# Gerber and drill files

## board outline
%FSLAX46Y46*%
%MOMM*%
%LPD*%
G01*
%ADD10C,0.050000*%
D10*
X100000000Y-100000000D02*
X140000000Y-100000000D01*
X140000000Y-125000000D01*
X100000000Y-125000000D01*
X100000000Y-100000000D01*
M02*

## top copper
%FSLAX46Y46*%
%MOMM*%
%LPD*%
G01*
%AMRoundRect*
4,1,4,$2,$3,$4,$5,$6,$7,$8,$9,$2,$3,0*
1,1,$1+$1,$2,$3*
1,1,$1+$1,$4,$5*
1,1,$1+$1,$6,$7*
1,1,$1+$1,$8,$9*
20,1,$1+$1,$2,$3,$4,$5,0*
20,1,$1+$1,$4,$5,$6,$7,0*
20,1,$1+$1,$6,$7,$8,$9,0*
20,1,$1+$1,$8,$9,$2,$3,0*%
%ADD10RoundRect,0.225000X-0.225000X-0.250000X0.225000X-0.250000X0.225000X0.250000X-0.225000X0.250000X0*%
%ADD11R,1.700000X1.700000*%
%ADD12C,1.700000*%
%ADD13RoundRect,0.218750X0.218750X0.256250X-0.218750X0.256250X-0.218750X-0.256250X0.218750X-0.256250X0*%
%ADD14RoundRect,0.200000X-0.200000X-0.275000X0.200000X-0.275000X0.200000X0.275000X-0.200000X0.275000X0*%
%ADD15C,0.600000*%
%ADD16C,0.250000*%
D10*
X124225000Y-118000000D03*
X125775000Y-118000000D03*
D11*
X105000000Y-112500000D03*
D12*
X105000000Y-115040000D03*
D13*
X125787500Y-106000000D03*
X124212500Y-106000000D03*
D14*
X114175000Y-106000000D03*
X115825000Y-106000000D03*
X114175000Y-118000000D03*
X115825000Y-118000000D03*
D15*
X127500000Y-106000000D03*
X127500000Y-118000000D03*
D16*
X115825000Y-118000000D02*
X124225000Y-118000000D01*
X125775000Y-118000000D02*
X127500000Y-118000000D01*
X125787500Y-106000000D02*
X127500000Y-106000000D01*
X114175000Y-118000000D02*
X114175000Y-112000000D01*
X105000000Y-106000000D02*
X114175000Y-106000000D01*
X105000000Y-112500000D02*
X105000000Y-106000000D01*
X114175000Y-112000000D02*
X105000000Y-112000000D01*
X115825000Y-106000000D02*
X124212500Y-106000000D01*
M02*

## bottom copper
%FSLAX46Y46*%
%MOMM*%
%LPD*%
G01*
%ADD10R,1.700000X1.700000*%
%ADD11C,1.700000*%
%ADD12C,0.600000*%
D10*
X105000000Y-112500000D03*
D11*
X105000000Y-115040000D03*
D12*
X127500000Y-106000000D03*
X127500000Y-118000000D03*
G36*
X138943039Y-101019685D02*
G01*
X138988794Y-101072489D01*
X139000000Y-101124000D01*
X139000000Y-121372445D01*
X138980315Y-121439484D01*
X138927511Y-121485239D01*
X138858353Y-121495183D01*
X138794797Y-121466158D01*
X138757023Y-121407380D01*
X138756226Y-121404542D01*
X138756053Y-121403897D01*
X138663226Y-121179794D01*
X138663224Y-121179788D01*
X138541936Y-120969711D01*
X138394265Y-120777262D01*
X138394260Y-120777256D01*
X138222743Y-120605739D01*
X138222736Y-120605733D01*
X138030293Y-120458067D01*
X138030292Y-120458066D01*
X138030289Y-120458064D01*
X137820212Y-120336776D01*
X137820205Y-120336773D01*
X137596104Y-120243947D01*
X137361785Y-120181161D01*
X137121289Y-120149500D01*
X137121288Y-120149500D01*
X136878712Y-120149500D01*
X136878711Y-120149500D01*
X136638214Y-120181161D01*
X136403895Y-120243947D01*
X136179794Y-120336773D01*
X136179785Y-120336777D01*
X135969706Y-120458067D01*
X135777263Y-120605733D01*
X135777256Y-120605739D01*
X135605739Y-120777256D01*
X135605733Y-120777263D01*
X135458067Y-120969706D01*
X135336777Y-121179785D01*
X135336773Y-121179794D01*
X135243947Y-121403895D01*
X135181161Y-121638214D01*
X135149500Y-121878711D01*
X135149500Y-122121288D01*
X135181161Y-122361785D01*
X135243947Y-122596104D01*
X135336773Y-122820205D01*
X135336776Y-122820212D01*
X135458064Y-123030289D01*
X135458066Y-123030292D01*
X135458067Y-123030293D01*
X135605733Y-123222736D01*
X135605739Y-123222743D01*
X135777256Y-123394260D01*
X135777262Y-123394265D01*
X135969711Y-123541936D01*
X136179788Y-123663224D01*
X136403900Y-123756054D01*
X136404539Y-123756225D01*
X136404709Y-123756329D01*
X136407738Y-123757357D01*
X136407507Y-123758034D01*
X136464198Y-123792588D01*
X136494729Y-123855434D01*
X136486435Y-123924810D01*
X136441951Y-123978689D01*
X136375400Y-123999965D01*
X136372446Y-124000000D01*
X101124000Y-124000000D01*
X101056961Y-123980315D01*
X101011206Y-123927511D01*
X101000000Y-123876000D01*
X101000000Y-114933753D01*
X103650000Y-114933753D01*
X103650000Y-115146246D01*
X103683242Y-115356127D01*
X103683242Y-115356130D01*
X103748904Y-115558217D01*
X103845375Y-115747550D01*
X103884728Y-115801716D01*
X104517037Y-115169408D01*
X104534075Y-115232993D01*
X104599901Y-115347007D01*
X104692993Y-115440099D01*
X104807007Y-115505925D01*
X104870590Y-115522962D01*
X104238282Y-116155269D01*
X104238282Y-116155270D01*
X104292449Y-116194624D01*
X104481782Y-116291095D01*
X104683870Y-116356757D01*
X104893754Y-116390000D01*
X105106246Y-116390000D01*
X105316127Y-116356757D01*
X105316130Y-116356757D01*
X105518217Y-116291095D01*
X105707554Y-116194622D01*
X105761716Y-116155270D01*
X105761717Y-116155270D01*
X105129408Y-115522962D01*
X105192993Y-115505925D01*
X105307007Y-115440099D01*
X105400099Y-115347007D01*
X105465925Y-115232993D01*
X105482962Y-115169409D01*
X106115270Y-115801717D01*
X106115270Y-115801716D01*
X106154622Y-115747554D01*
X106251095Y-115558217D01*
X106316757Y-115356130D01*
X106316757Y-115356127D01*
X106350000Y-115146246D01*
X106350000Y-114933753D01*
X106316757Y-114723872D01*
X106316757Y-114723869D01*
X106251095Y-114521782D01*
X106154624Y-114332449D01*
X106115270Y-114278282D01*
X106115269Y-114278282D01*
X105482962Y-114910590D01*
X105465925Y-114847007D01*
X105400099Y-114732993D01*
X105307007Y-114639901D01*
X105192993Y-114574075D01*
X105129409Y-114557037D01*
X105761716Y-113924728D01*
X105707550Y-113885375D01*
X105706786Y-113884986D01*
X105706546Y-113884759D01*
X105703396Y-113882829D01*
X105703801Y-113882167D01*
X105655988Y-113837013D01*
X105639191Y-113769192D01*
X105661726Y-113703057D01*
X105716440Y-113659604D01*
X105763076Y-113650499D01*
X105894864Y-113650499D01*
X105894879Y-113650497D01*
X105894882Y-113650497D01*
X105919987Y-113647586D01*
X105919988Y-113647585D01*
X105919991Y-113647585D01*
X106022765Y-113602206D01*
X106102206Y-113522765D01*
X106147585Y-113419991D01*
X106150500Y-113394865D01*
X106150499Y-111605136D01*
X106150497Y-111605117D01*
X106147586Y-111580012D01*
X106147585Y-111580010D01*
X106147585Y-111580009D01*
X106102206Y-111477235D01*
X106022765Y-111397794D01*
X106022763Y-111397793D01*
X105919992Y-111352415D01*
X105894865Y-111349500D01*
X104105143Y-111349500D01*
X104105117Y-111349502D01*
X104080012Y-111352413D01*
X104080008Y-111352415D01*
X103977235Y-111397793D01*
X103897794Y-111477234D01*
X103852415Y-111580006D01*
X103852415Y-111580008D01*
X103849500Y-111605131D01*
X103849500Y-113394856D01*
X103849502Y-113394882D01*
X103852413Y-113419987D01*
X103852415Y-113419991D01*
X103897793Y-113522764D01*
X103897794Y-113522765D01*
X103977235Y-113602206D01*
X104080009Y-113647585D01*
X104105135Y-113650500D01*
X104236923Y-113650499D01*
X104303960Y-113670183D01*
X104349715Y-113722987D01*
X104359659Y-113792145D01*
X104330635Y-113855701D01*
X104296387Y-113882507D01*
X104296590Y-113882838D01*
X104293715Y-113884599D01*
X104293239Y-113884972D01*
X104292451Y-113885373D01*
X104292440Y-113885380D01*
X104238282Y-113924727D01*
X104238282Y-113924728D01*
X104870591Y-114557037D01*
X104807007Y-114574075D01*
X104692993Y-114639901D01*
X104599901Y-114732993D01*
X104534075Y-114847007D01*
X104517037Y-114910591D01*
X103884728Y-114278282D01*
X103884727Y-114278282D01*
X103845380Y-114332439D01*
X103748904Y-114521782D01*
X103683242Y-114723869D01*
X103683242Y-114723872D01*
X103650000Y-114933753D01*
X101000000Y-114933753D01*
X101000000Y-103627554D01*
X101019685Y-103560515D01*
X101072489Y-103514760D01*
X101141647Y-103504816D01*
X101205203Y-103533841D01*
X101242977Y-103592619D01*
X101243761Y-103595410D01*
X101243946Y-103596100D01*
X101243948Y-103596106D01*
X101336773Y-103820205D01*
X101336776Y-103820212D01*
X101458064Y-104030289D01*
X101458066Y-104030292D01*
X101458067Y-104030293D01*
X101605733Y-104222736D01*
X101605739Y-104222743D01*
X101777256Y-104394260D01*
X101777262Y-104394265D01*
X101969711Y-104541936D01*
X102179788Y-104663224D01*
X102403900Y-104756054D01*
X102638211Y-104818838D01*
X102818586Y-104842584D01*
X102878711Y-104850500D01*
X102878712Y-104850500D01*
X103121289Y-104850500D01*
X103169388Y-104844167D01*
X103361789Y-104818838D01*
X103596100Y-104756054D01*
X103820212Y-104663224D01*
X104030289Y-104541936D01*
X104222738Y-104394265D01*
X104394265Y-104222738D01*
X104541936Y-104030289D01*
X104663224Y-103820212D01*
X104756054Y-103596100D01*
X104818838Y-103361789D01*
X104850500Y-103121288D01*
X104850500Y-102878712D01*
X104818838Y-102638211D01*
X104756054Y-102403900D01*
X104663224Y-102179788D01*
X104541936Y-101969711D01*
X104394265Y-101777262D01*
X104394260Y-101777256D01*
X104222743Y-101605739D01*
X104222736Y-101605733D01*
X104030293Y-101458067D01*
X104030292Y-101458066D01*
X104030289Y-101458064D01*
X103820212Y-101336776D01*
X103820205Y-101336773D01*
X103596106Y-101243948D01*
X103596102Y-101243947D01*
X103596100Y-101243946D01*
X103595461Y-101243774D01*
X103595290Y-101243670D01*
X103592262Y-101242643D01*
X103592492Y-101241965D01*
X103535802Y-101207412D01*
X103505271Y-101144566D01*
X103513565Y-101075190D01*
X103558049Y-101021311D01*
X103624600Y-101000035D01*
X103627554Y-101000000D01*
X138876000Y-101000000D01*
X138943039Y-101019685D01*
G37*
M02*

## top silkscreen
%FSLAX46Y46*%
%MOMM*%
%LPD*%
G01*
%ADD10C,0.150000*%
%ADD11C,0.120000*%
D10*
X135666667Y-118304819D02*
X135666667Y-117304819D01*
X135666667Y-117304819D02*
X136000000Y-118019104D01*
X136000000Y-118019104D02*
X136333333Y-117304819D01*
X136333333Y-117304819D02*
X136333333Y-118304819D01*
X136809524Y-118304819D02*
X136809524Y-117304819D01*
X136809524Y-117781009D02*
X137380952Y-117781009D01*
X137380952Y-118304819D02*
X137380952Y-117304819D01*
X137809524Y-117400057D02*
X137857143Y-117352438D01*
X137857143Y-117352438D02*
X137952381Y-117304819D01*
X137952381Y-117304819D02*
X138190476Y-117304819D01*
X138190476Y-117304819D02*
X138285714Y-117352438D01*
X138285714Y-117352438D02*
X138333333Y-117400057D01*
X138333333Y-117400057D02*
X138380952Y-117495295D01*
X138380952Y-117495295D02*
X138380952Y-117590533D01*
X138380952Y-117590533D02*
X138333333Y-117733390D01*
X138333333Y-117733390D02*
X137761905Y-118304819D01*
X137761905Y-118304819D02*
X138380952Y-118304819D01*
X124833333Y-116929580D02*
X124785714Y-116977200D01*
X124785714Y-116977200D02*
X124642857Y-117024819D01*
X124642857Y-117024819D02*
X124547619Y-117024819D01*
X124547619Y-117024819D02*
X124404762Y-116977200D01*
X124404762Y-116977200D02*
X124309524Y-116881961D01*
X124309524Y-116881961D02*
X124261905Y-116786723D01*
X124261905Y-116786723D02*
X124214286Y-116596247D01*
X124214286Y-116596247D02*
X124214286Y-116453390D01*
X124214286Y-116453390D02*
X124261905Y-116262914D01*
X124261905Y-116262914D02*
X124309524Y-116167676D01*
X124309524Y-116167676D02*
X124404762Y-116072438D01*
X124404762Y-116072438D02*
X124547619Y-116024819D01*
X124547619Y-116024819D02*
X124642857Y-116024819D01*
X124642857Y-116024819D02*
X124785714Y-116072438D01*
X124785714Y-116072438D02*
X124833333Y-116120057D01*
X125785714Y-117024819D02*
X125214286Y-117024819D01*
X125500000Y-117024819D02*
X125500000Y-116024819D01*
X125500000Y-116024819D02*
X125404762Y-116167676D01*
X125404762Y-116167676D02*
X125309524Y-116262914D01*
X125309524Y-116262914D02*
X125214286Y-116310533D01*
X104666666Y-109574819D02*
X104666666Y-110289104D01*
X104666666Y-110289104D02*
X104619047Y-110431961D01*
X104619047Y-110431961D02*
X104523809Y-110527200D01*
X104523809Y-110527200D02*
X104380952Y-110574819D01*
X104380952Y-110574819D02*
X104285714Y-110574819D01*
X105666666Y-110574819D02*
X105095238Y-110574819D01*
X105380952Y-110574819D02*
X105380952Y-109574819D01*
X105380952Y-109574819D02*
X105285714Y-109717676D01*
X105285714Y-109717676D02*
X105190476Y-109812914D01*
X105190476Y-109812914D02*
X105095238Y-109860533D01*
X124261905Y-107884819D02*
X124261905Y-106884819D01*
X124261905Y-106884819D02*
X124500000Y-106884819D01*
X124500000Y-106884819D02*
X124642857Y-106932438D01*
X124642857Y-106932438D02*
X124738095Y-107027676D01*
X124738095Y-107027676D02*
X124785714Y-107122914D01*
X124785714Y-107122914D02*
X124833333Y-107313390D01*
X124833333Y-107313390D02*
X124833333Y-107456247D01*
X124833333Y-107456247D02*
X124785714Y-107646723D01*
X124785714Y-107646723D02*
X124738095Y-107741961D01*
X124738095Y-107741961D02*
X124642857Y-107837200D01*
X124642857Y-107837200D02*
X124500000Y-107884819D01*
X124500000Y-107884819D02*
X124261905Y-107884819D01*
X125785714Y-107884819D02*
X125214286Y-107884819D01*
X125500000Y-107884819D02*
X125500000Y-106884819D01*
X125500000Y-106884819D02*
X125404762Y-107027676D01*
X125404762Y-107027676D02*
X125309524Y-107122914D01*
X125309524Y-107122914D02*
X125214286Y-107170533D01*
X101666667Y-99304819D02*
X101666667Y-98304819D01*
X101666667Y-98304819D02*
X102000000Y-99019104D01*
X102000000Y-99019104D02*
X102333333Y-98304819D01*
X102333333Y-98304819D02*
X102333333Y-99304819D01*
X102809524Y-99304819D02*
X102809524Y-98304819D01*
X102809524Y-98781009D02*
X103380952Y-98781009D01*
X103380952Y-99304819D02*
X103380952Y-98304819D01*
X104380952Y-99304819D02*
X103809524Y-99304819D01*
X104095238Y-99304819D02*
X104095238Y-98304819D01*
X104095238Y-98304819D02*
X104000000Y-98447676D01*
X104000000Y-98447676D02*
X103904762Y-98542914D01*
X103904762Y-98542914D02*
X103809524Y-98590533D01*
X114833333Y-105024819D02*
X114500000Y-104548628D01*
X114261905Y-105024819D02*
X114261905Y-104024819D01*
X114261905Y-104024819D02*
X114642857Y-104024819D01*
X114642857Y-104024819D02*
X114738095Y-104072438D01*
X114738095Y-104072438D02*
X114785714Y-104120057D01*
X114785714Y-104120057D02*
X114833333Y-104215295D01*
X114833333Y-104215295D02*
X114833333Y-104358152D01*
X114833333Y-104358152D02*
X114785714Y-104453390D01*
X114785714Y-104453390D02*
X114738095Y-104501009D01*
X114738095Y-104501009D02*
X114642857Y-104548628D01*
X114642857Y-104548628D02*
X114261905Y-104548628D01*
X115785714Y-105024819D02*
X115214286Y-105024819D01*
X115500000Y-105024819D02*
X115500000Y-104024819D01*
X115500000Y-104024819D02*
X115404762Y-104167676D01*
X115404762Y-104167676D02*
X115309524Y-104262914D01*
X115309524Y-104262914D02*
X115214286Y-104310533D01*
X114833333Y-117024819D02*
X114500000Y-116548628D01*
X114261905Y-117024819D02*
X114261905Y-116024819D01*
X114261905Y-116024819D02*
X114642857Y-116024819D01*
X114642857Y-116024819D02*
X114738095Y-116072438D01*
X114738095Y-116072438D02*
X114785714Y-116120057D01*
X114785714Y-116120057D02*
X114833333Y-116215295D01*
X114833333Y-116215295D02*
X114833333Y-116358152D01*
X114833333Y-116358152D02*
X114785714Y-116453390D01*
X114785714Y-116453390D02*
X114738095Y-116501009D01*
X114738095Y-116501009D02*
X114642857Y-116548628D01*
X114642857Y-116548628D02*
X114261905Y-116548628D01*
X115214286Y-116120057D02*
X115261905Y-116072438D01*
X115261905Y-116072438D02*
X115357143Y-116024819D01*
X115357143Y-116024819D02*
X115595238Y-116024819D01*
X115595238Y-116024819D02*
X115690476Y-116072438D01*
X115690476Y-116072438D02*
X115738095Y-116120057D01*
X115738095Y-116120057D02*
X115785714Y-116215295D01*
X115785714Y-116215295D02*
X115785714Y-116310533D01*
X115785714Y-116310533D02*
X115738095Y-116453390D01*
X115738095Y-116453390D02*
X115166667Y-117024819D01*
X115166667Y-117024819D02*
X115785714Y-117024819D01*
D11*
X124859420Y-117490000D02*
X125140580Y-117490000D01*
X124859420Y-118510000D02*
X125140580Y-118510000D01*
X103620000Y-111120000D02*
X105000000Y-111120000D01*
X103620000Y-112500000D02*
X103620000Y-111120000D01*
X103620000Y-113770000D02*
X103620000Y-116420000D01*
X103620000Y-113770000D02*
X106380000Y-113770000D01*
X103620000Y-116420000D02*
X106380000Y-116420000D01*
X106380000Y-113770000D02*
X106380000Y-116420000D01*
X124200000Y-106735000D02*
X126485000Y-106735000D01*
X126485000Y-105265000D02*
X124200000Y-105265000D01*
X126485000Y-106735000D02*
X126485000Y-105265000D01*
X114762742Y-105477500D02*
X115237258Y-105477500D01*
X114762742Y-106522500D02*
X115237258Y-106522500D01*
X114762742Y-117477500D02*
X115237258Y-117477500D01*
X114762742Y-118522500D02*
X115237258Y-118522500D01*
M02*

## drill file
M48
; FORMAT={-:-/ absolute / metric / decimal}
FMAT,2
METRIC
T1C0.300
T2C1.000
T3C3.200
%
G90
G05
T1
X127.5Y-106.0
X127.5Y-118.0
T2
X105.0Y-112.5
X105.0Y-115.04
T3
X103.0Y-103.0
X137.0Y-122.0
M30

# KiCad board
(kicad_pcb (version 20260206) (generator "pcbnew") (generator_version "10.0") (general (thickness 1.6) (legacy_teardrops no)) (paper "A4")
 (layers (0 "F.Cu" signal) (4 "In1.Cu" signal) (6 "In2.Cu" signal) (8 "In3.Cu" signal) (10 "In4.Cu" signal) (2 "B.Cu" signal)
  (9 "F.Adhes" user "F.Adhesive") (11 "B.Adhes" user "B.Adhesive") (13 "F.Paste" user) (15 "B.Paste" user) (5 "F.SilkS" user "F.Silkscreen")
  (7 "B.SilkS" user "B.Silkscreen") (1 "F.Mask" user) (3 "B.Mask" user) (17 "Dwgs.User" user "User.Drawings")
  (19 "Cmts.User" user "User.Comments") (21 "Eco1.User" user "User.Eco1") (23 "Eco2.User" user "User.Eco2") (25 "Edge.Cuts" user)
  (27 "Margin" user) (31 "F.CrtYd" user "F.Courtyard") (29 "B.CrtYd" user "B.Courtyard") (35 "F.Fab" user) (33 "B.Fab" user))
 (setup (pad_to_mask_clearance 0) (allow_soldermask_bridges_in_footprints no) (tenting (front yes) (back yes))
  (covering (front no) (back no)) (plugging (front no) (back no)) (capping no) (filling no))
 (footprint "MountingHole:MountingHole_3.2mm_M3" (layer "F.Cu") (at 137 122)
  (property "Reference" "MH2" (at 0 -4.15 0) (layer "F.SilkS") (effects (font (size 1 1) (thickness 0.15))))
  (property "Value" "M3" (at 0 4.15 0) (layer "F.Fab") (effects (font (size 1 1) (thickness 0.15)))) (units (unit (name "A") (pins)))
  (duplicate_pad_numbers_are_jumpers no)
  (pad "" np_thru_hole circle (at 0 0) (size 3.2 3.2) (drill 3.2) (layers "*.Cu" "*.Mask")))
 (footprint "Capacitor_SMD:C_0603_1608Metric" (layer "F.Cu") (at 125 118)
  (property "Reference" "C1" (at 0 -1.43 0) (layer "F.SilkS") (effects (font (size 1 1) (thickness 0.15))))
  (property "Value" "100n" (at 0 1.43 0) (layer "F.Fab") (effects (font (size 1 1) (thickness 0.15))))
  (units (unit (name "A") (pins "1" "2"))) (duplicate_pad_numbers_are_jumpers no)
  (fp_line (start -0.14058 -0.51) (end 0.14058 -0.51) (stroke (width 0.12) (type solid)) (layer "F.SilkS"))
  (fp_line (start -0.14058 0.51) (end 0.14058 0.51) (stroke (width 0.12) (type solid)) (layer "F.SilkS"))
  (pad "1" smd roundrect (at -0.775 0) (size 0.9 0.95) (layers "F.Cu" "F.Mask" "F.Paste") (roundrect_rratio 0.25) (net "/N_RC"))
  (pad "2" smd roundrect (at 0.775 0) (size 0.9 0.95) (layers "F.Cu" "F.Mask" "F.Paste") (roundrect_rratio 0.25) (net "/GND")))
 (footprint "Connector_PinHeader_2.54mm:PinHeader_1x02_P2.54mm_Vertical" (layer "F.Cu") (at 105 112.5)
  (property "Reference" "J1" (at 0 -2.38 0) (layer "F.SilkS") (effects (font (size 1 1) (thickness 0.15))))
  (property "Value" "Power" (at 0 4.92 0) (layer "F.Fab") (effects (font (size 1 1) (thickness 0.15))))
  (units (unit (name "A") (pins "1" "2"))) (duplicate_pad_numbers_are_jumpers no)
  (fp_line (start -1.38 -1.38) (end 0 -1.38) (stroke (width 0.12) (type solid)) (layer "F.SilkS"))
  (fp_line (start -1.38 0) (end -1.38 -1.38) (stroke (width 0.12) (type solid)) (layer "F.SilkS"))
  (fp_line (start -1.38 1.27) (end -1.38 3.92) (stroke (width 0.12) (type solid)) (layer "F.SilkS"))
  (fp_line (start -1.38 1.27) (end 1.38 1.27) (stroke (width 0.12) (type solid)) (layer "F.SilkS"))
  (fp_line (start -1.38 3.92) (end 1.38 3.92) (stroke (width 0.12) (type solid)) (layer "F.SilkS"))
  (fp_line (start 1.38 1.27) (end 1.38 3.92) (stroke (width 0.12) (type solid)) (layer "F.SilkS"))
  (pad "1" thru_hole rect (at 0 0) (size 1.7 1.7) (drill 1) (layers "*.Cu" "*.Mask") (remove_unused_layers no) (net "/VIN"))
  (pad "2" thru_hole circle (at 0 2.54) (size 1.7 1.7) (drill 1) (layers "*.Cu" "*.Mask") (remove_unused_layers no) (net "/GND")))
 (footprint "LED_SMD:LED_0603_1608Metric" (layer "F.Cu") (at 125 106 180)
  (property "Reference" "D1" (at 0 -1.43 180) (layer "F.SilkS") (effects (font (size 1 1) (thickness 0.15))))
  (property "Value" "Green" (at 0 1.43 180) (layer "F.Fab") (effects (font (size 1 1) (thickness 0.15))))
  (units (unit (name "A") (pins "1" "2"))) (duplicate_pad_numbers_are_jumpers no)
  (fp_line (start 0.8 -0.735) (end -1.485 -0.735) (stroke (width 0.12) (type solid)) (layer "F.SilkS"))
  (fp_line (start -1.485 0.735) (end 0.8 0.735) (stroke (width 0.12) (type solid)) (layer "F.SilkS"))
  (fp_line (start -1.485 -0.735) (end -1.485 0.735) (stroke (width 0.12) (type solid)) (layer "F.SilkS"))
  (pad "1" smd roundrect (at -0.7875 0 180) (size 0.875 0.95) (layers "F.Cu" "F.Mask" "F.Paste") (roundrect_rratio 0.25) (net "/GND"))
  (pad "2" smd roundrect (at 0.7875 0 180) (size 0.875 0.95) (layers "F.Cu" "F.Mask" "F.Paste") (roundrect_rratio 0.25) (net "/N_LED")))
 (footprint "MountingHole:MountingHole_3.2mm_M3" (layer "F.Cu") (at 103 103)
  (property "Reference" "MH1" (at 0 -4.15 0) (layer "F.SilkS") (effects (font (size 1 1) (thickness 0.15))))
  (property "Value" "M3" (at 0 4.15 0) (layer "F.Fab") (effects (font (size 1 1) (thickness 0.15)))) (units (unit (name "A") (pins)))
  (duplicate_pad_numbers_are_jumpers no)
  (pad "" np_thru_hole circle (at 0 0) (size 3.2 3.2) (drill 3.2) (layers "*.Cu" "*.Mask")))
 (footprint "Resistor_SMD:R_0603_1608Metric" (layer "F.Cu") (at 115 106)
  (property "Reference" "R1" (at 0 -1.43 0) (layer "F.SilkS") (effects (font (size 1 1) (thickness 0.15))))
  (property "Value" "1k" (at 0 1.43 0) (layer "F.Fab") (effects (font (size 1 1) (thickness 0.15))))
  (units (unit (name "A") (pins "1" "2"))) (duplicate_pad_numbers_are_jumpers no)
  (fp_line (start -0.237258 -0.5225) (end 0.237258 -0.5225) (stroke (width 0.12) (type solid)) (layer "F.SilkS"))
  (fp_line (start -0.237258 0.5225) (end 0.237258 0.5225) (stroke (width 0.12) (type solid)) (layer "F.SilkS"))
  (pad "1" smd roundrect (at -0.825 0) (size 0.8 0.95) (layers "F.Cu" "F.Mask" "F.Paste") (roundrect_rratio 0.25) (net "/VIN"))
  (pad "2" smd roundrect (at 0.825 0) (size 0.8 0.95) (layers "F.Cu" "F.Mask" "F.Paste") (roundrect_rratio 0.25) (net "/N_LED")))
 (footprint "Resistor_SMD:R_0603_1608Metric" (layer "F.Cu") (at 115 118)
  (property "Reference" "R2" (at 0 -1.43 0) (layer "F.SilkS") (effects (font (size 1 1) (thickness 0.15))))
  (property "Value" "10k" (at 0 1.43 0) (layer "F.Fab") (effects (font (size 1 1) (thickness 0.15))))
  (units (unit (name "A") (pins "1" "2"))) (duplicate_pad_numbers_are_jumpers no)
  (fp_line (start -0.237258 -0.5225) (end 0.237258 -0.5225) (stroke (width 0.12) (type solid)) (layer "F.SilkS"))
  (fp_line (start -0.237258 0.5225) (end 0.237258 0.5225) (stroke (width 0.12) (type solid)) (layer "F.SilkS"))
  (pad "1" smd roundrect (at -0.825 0) (size 0.8 0.95) (layers "F.Cu" "F.Mask" "F.Paste") (roundrect_rratio 0.25) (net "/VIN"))
  (pad "2" smd roundrect (at 0.825 0) (size 0.8 0.95) (layers "F.Cu" "F.Mask" "F.Paste") (roundrect_rratio 0.25) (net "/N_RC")))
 (gr_rect (start 100 100) (end 140 125) (stroke (width 0.05) (type default)) (fill no) (layer "Edge.Cuts"))
 (segment (start 115.825 118) (end 124.225 118) (width 0.25) (layer "F.Cu") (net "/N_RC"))
 (segment (start 125.775 118) (end 127.5 118) (width 0.25) (layer "F.Cu") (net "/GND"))
 (segment (start 125.7875 106) (end 127.5 106) (width 0.25) (layer "F.Cu") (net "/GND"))
 (via (at 127.5 106) (size 0.6) (drill 0.3) (layers "F.Cu" "B.Cu") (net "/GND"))
 (via (at 127.5 118) (size 0.6) (drill 0.3) (layers "F.Cu" "B.Cu") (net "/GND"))
 (segment (start 114.175 118) (end 114.175 112) (width 0.25) (layer "F.Cu") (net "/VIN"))
 (segment (start 105 106) (end 114.175 106) (width 0.25) (layer "F.Cu") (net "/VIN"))
 (segment (start 105 112.5) (end 105 106) (width 0.25) (layer "F.Cu") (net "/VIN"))
 (segment (start 114.175 112) (end 105 112) (width 0.25) (layer "F.Cu") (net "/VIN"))
 (segment (start 115.825 106) (end 124.2125 106) (width 0.25) (layer "F.Cu") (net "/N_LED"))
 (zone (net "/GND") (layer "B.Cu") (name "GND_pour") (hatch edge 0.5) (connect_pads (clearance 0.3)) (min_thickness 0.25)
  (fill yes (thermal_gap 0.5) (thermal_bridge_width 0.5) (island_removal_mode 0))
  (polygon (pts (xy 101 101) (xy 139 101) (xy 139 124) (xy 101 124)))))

